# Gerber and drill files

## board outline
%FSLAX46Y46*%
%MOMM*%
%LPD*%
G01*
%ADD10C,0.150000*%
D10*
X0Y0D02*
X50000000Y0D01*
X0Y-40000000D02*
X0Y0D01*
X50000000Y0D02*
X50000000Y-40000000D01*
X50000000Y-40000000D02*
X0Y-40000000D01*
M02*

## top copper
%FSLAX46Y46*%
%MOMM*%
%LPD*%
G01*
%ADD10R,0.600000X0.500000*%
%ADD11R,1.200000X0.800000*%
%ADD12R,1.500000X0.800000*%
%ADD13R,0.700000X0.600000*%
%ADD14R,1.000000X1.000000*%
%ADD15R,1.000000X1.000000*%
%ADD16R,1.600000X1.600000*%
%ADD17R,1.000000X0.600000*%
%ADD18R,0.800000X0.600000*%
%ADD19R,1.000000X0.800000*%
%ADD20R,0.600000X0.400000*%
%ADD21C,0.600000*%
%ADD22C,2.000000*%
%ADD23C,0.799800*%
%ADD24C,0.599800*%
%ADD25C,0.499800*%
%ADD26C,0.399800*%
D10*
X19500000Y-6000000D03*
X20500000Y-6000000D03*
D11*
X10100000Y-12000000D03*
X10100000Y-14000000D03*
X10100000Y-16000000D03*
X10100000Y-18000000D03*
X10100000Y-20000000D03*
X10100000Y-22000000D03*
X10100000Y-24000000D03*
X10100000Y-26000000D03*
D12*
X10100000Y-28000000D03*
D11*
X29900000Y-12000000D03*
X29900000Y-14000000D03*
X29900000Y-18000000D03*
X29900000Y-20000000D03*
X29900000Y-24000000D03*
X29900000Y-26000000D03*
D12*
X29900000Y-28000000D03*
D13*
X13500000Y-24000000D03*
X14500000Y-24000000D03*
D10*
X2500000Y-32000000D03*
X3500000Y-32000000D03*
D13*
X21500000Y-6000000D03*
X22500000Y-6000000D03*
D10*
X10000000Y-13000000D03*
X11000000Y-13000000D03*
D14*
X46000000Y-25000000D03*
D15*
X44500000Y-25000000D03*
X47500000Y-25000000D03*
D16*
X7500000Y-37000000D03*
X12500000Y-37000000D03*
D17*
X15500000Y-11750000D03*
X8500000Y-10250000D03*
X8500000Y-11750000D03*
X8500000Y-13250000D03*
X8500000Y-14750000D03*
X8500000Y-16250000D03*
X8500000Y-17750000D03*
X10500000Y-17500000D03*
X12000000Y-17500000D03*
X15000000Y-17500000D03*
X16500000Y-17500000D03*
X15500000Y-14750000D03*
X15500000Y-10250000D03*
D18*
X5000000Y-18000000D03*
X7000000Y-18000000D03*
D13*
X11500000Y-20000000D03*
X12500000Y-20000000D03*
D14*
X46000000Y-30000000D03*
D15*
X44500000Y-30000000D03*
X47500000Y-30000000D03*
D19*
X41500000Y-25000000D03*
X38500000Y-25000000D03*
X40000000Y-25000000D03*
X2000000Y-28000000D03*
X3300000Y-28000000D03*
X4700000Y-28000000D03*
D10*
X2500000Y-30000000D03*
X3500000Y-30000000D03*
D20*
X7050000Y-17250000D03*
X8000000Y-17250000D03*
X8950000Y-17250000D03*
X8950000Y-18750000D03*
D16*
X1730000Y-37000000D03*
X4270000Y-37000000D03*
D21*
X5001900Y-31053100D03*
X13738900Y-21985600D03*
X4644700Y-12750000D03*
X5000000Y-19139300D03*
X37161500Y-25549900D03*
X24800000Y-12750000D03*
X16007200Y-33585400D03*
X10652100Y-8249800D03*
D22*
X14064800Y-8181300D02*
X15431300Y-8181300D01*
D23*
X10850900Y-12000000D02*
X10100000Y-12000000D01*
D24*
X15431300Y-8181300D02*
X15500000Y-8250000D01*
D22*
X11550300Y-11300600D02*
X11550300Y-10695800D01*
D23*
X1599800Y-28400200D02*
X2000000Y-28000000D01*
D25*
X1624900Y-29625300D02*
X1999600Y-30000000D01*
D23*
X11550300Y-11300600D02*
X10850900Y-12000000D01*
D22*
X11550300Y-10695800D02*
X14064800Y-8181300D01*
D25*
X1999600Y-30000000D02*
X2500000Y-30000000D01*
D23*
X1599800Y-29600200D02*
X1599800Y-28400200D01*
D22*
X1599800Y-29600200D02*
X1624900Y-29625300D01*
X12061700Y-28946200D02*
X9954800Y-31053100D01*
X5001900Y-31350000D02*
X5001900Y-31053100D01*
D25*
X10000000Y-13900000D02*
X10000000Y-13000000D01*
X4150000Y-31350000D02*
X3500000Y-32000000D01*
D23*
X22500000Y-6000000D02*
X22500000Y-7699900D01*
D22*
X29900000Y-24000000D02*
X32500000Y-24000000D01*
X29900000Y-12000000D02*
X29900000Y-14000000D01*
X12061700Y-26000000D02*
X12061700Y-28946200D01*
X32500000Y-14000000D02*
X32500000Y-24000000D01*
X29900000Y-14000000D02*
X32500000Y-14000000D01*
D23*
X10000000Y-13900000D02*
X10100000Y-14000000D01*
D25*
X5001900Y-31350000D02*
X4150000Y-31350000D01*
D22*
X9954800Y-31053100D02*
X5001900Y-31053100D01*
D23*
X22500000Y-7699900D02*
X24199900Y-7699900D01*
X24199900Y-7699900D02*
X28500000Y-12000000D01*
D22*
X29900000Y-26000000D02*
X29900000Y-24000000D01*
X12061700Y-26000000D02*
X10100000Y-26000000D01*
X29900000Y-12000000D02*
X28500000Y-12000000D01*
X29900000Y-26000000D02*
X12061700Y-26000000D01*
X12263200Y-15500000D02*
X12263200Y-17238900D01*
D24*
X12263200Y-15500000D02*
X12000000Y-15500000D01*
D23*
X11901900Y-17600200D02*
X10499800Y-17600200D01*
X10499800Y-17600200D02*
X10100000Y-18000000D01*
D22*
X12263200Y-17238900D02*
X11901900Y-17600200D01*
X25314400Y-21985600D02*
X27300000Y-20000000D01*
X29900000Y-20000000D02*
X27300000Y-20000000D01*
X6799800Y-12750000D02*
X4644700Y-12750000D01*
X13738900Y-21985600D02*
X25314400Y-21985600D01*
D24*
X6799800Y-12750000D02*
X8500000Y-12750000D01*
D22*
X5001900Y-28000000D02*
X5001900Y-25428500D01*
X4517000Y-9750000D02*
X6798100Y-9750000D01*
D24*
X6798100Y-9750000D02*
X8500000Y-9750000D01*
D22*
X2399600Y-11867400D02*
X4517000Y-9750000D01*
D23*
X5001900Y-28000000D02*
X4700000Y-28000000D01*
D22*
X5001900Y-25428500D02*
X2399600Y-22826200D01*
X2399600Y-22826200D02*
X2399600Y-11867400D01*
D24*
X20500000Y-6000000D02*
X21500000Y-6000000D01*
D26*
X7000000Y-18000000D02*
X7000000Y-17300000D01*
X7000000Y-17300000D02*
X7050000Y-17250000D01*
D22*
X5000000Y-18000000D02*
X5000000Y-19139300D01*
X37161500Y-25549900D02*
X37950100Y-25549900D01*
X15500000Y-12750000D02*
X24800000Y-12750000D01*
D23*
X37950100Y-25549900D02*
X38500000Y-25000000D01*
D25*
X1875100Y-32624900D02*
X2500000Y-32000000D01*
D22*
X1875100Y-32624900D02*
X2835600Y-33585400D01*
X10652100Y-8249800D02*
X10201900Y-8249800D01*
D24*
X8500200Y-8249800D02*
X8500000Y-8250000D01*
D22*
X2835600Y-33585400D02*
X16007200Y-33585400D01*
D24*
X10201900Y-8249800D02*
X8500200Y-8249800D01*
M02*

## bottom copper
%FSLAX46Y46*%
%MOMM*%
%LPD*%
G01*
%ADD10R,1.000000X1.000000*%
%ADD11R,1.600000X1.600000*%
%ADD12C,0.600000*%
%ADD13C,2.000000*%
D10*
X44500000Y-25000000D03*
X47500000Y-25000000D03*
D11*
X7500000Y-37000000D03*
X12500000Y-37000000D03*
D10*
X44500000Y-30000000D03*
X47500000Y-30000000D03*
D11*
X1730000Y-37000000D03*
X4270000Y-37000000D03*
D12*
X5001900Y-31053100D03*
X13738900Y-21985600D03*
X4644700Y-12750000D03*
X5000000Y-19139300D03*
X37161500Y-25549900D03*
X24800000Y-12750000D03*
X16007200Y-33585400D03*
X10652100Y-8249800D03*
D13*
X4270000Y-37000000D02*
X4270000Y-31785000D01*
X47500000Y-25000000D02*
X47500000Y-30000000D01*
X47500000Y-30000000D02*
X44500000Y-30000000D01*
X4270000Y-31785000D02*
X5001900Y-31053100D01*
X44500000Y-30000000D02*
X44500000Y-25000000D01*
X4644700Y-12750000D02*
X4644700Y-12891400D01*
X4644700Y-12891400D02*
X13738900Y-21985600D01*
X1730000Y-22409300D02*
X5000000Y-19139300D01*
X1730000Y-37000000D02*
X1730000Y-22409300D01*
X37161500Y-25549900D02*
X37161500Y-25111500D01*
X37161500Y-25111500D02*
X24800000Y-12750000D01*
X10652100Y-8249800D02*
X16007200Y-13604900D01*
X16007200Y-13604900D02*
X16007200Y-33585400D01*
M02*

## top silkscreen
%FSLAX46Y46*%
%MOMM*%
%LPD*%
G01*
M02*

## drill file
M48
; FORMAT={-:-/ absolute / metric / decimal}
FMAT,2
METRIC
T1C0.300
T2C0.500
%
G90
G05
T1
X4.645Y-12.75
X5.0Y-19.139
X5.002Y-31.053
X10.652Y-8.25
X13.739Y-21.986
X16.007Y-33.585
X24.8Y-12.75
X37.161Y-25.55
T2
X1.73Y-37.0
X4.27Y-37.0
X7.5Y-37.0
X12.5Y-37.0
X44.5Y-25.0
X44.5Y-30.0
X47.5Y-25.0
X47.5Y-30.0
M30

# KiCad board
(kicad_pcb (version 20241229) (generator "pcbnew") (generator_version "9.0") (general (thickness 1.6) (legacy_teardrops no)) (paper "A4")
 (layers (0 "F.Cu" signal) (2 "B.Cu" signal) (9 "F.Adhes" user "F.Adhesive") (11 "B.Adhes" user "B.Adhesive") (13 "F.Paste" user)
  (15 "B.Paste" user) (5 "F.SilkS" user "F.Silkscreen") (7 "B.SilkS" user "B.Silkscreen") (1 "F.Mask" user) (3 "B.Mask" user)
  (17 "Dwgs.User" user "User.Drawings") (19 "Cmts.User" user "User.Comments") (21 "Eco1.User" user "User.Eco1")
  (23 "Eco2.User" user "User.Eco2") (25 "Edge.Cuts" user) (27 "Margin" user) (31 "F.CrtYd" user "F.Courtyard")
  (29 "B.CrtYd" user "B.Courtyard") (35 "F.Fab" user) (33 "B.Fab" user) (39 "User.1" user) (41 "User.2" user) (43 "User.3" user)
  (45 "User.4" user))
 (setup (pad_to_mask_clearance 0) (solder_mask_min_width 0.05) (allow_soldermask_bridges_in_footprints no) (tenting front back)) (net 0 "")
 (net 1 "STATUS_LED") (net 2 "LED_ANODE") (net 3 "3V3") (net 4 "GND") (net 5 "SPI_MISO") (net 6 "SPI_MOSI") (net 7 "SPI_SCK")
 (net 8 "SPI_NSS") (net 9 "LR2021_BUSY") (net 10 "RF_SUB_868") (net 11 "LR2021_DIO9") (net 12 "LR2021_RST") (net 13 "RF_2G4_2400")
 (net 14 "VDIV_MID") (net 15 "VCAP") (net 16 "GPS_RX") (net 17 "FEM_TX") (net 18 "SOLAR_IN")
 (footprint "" (layer "F.Cu") (at 20 6)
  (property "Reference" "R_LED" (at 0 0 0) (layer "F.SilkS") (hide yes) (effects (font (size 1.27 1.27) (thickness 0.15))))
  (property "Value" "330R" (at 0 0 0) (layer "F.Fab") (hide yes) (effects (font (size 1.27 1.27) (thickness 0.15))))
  (pad "1" smd rect (at -0.5 0) (size 0.6 0.5) (layers "F.Cu" "F.Mask") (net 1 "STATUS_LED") (thermal_bridge_angle 45))
  (pad "2" smd rect (at 0.5 0) (size 0.6 0.5) (layers "F.Cu" "F.Mask") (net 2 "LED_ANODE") (thermal_bridge_angle 45)))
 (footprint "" (layer "F.Cu") (at 20 20)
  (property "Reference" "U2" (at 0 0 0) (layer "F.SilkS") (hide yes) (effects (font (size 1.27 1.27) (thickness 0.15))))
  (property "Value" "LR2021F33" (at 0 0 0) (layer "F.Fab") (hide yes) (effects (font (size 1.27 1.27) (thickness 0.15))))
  (pad "1" smd rect (at -9.9 -8) (size 1.2 0.8) (layers "F.Cu" "F.Mask") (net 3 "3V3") (thermal_bridge_angle 45))
  (pad "2" smd rect (at -9.9 -6) (size 1.2 0.8) (layers "F.Cu" "F.Mask") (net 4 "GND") (thermal_bridge_angle 45))
  (pad "3" smd rect (at -9.9 -4) (size 1.2 0.8) (layers "F.Cu" "F.Mask") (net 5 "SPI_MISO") (thermal_bridge_angle 45))
  (pad "4" smd rect (at -9.9 -2) (size 1.2 0.8) (layers "F.Cu" "F.Mask") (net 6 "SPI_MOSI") (thermal_bridge_angle 45))
  (pad "5" smd rect (at -9.9 0) (size 1.2 0.8) (layers "F.Cu" "F.Mask") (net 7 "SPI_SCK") (thermal_bridge_angle 45))
  (pad "6" smd rect (at -9.9 2) (size 1.2 0.8) (layers "F.Cu" "F.Mask") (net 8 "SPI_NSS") (thermal_bridge_angle 45))
  (pad "7" smd rect (at -9.9 4) (size 1.2 0.8) (layers "F.Cu" "F.Mask") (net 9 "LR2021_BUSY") (thermal_bridge_angle 45))
  (pad "8" smd rect (at -9.9 6) (size 1.2 0.8) (layers "F.Cu" "F.Mask") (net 4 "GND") (thermal_bridge_angle 45))
  (pad "9" smd rect (at -9.9 8) (size 1.5 0.8) (layers "F.Cu" "F.Mask") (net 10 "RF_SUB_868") (thermal_bridge_angle 45))
  (pad "10" smd rect (at 9.9 -8) (size 1.2 0.8) (layers "F.Cu" "F.Mask") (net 4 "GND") (thermal_bridge_angle 45))
  (pad "11" smd rect (at 9.9 -6) (size 1.2 0.8) (layers "F.Cu" "F.Mask") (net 4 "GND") (thermal_bridge_angle 45))
  (pad "13" smd rect (at 9.9 -2) (size 1.2 0.8) (layers "F.Cu" "F.Mask") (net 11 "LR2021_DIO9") (thermal_bridge_angle 45))
  (pad "14" smd rect (at 9.9 0) (size 1.2 0.8) (layers "F.Cu" "F.Mask") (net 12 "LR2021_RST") (thermal_bridge_angle 45))
  (pad "16" smd rect (at 9.9 4) (size 1.2 0.8) (layers "F.Cu" "F.Mask") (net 4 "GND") (thermal_bridge_angle 45))
  (pad "17" smd rect (at 9.9 6) (size 1.2 0.8) (layers "F.Cu" "F.Mask") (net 4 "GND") (thermal_bridge_angle 45))
  (pad "18" smd rect (at 9.9 8) (size 1.5 0.8) (layers "F.Cu" "F.Mask") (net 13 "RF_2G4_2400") (thermal_bridge_angle 45)))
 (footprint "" (layer "F.Cu") (at 14 24)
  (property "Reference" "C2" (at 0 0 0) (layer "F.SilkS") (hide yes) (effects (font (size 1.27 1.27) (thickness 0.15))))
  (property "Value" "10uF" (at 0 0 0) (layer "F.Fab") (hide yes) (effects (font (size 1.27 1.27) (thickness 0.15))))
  (pad "1" smd rect (at -0.5 0) (size 0.7 0.6) (layers "F.Cu" "F.Mask") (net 3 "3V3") (thermal_bridge_angle 45))
  (pad "2" smd rect (at 0.5 0) (size 0.7 0.6) (layers "F.Cu" "F.Mask") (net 4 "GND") (thermal_bridge_angle 45)))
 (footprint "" (layer "F.Cu") (at 3 32)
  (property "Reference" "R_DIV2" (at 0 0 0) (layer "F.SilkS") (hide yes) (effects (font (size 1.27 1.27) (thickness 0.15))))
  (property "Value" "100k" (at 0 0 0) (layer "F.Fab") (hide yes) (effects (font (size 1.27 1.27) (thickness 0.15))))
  (pad "1" smd rect (at -0.5 0) (size 0.6 0.5) (layers "F.Cu" "F.Mask") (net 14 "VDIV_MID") (thermal_bridge_angle 45))
  (pad "2" smd rect (at 0.5 0) (size 0.6 0.5) (layers "F.Cu" "F.Mask") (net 4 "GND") (thermal_bridge_angle 45)))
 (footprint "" (layer "F.Cu") (at 22 6)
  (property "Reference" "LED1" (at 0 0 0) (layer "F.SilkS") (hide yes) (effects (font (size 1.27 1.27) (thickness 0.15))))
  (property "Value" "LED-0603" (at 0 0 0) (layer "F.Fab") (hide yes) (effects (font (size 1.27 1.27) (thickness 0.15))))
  (pad "A" smd rect (at -0.5 0) (size 0.7 0.6) (layers "F.Cu" "F.Mask") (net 2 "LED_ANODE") (thermal_bridge_angle 45))
  (pad "K" smd rect (at 0.5 0) (size 0.7 0.6) (layers "F.Cu" "F.Mask") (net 4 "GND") (thermal_bridge_angle 45)))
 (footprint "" (layer "F.Cu") (at 10.5 13)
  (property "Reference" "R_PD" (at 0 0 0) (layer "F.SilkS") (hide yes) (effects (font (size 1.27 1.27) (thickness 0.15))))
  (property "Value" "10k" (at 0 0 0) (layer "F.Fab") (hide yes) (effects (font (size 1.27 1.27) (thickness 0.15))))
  (pad "1" smd rect (at -0.5 0) (size 0.6 0.5) (layers "F.Cu" "F.Mask") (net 4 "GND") (thermal_bridge_angle 45))
  (pad "2" smd rect (at 0.5 0) (size 0.6 0.5) (layers "F.Cu" "F.Mask") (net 5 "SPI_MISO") (thermal_bridge_angle 45)))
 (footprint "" (layer "F.Cu") (at 46 25)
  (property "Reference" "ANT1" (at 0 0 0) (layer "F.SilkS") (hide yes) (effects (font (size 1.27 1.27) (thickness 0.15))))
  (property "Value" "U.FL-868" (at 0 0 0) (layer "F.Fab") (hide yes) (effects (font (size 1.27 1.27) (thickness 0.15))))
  (pad "1" smd rect (at 0 0) (size 1 1) (layers "F.Cu" "F.Mask") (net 10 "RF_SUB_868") (thermal_bridge_angle 45))
  (pad "2" thru_hole rect (at -1.5 0) (size 1 1) (drill 0.5) (layers "*.Cu" "*.Mask") (remove_unused_layers no) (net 4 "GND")
   (thermal_bridge_angle 45))
  (pad "3" thru_hole rect (at 1.5 0) (size 1 1) (drill 0.5) (layers "*.Cu" "*.Mask") (remove_unused_layers no) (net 4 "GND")
   (thermal_bridge_angle 45)))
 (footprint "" (layer "F.Cu") (at 10 37)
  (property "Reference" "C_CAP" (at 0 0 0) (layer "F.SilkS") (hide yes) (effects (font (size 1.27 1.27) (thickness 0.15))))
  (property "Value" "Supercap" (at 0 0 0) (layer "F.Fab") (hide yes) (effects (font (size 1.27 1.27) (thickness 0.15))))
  (pad "1" thru_hole rect (at -2.5 0) (size 1.6 1.6) (drill 0.5) (layers "*.Cu" "*.Mask") (remove_unused_layers no) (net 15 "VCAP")
   (thermal_bridge_angle 45))
  (pad "2" thru_hole rect (at 2.5 0) (size 1.6 1.6) (drill 0.5) (layers "*.Cu" "*.Mask") (remove_unused_layers no) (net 4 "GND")
   (thermal_bridge_angle 45)))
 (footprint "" (layer "F.Cu") (at 12 14)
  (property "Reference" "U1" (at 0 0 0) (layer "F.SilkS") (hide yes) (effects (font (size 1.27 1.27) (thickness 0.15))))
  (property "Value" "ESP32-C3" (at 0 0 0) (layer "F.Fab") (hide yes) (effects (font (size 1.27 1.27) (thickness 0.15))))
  (pad "GND" smd rect (at 3.5 -2.25) (size 1 0.6) (layers "F.Cu" "F.Mask") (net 4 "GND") (thermal_bridge_angle 45))
  (pad "GPIO0" smd rect (at -3.5 -3.75) (size 1 0.6) (layers "F.Cu" "F.Mask") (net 14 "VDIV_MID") (thermal_bridge_angle 45))
  (pad "GPIO1" smd rect (at -3.5 -2.25) (size 1 0.6) (layers "F.Cu" "F.Mask") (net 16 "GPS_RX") (thermal_bridge_angle 45))
  (pad "GPIO2" smd rect (at -3.5 -0.75) (size 1 0.6) (layers "F.Cu" "F.Mask") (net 5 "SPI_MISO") (thermal_bridge_angle 45))
  (pad "GPIO3" smd rect (at -3.5 0.75) (size 1 0.6) (layers "F.Cu" "F.Mask") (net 12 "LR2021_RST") (thermal_bridge_angle 45))
  (pad "GPIO4" smd rect (at -3.5 2.25) (size 1 0.6) (layers "F.Cu" "F.Mask") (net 9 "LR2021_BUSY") (thermal_bridge_angle 45))
  (pad "GPIO5" smd rect (at -3.5 3.75) (size 1 0.6) (layers "F.Cu" "F.Mask") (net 11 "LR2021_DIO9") (thermal_bridge_angle 45))
  (pad "GPIO6" smd rect (at -1.5 3.5) (size 1 0.6) (layers "F.Cu" "F.Mask") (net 7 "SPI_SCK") (thermal_bridge_angle 45))
  (pad "GPIO7" smd rect (at 0 3.5) (size 1 0.6) (layers "F.Cu" "F.Mask") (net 6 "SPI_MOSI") (thermal_bridge_angle 45))
  (pad "GPIO9" smd rect (at 3 3.5) (size 1 0.6) (layers "F.Cu" "F.Mask") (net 1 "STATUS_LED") (thermal_bridge_angle 45))
  (pad "GPIO10" smd rect (at 4.5 3.5) (size 1 0.6) (layers "F.Cu" "F.Mask") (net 8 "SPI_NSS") (thermal_bridge_angle 45))
  (pad "GPIO19" smd rect (at 3.5 0.75) (size 1 0.6) (layers "F.Cu" "F.Mask") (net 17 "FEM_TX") (thermal_bridge_angle 45))
  (pad "VCC" smd rect (at 3.5 -3.75) (size 1 0.6) (layers "F.Cu" "F.Mask") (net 3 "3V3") (thermal_bridge_angle 45)))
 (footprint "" (layer "F.Cu") (at 6 18)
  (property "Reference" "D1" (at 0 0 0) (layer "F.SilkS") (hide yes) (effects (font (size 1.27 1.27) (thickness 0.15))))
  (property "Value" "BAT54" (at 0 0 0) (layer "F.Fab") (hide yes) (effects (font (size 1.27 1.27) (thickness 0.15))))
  (pad "A" smd rect (at -1 0) (size 0.8 0.6) (layers "F.Cu" "F.Mask") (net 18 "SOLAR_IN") (thermal_bridge_angle 45))
  (pad "K" smd rect (at 1 0) (size 0.8 0.6) (layers "F.Cu" "F.Mask") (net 15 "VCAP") (thermal_bridge_angle 45)))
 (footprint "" (layer "F.Cu") (at 12 20)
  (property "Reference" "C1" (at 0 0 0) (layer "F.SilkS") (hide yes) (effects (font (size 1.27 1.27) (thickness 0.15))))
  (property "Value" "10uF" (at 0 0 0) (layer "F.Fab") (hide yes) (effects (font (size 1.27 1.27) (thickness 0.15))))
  (pad "1" smd rect (at -0.5 0) (size 0.7 0.6) (layers "F.Cu" "F.Mask") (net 15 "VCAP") (thermal_bridge_angle 45))
  (pad "2" smd rect (at 0.5 0) (size 0.7 0.6) (layers "F.Cu" "F.Mask") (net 4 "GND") (thermal_bridge_angle 45)))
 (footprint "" (layer "F.Cu") (at 46 30)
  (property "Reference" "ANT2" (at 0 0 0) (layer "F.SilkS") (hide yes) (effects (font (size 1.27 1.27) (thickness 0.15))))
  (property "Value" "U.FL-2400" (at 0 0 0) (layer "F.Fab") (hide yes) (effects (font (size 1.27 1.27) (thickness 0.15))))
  (pad "1" smd rect (at 0 0) (size 1 1) (layers "F.Cu" "F.Mask") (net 13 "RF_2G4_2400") (thermal_bridge_angle 45))
  (pad "2" thru_hole rect (at -1.5 0) (size 1 1) (drill 0.5) (layers "*.Cu" "*.Mask") (remove_unused_layers no) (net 4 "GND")
   (thermal_bridge_angle 45))
  (pad "3" thru_hole rect (at 1.5 0) (size 1 1) (drill 0.5) (layers "*.Cu" "*.Mask") (remove_unused_layers no) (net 4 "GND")
   (thermal_bridge_angle 45)))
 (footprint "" (layer "F.Cu") (at 40 25)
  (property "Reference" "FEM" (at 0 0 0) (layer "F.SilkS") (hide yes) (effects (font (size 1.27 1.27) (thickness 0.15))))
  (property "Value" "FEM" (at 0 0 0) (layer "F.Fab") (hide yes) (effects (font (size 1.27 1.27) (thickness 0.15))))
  (pad "GND" smd rect (at 1.5 0) (size 1 0.8) (layers "F.Cu" "F.Mask") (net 4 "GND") (thermal_bridge_angle 45))
  (pad "TX" smd rect (at -1.5 0) (size 1 0.8) (layers "F.Cu" "F.Mask") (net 17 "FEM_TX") (thermal_bridge_angle 45))
  (pad "VCC" smd rect (at 0 0) (size 1 0.8) (layers "F.Cu" "F.Mask") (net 3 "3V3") (thermal_bridge_angle 45)))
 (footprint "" (layer "F.Cu") (at 4 28)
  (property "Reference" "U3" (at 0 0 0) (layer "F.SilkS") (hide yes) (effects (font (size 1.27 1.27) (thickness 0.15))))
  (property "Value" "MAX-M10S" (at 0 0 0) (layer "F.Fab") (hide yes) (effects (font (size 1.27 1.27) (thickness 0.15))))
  (pad "1" smd rect (at -2 0) (size 1 0.8) (layers "F.Cu" "F.Mask") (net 3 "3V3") (thermal_bridge_angle 45))
  (pad "2" smd rect (at -0.7 0) (size 1 0.8) (layers "F.Cu" "F.Mask") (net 4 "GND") (thermal_bridge_angle 45))
  (pad "3" smd rect (at 0.7 0) (size 1 0.8) (layers "F.Cu" "F.Mask") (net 16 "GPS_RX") (thermal_bridge_angle 45)))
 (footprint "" (layer "F.Cu") (at 3 30)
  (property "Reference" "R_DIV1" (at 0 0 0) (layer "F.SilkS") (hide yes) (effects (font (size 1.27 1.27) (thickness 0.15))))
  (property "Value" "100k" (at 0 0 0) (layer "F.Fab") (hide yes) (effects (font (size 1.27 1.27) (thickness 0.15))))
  (pad "1" smd rect (at -0.5 0) (size 0.6 0.5) (layers "F.Cu" "F.Mask") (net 3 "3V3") (thermal_bridge_angle 45))
  (pad "2" smd rect (at 0.5 0) (size 0.6 0.5) (layers "F.Cu" "F.Mask") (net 14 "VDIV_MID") (thermal_bridge_angle 45)))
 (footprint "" (layer "F.Cu") (at 8 18)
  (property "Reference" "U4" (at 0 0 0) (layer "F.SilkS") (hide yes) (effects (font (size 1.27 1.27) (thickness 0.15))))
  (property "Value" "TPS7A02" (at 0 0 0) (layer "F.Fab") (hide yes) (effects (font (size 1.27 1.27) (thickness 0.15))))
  (pad "1" smd rect (at -0.95 -0.75) (size 0.6 0.4) (layers "F.Cu" "F.Mask") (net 15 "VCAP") (thermal_bridge_angle 45))
  (pad "2" smd rect (at 0 -0.75) (size 0.6 0.4) (layers "F.Cu" "F.Mask") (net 4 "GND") (thermal_bridge_angle 45))
  (pad "3" smd rect (at 0.95 -0.75) (size 0.6 0.4) (layers "F.Cu" "F.Mask") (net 15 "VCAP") (thermal_bridge_angle 45))
  (pad "4" smd rect (at 0.95 0.75) (size 0.6 0.4) (layers "F.Cu" "F.Mask") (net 3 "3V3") (thermal_bridge_angle 45)))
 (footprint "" (layer "F.Cu") (at 3 37)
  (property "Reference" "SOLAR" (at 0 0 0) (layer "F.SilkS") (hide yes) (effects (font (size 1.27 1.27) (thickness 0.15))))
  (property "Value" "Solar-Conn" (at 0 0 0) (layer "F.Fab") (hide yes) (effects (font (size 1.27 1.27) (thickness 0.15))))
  (pad "1" thru_hole rect (at -1.27 0) (size 1.6 1.6) (drill 0.5) (layers "*.Cu" "*.Mask") (remove_unused_layers no) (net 18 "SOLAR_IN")
   (thermal_bridge_angle 45))
  (pad "2" thru_hole rect (at 1.27 0) (size 1.6 1.6) (drill 0.5) (layers "*.Cu" "*.Mask") (remove_unused_layers no) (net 4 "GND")
   (thermal_bridge_angle 45)))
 (gr_line (start 0 0) (end 50 0) (stroke (width 0.15) (type default)) (layer "Edge.Cuts"))
 (gr_line (start 0 40) (end 0 0) (stroke (width 0.15) (type default)) (layer "Edge.Cuts"))
 (gr_line (start 50 0) (end 50 40) (stroke (width 0.15) (type default)) (layer "Edge.Cuts"))
 (gr_line (start 50 40) (end 0 40) (stroke (width 0.15) (type default)) (layer "Edge.Cuts"))
 (segment (start 14.0648 8.1813) (end 15.4313 8.1813) (width 2) (layer "F.Cu") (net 3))
 (segment (start 10.8509 12) (end 10.1 12) (width 0.7998) (layer "F.Cu") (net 3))
 (segment (start 15.4313 8.1813) (end 15.5 8.25) (width 0.5998) (layer "F.Cu") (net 3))
 (segment (start 11.5503 11.3006) (end 11.5503 10.6958) (width 2) (layer "F.Cu") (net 3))
 (segment (start 1.5998 28.4002) (end 2 28) (width 0.7998) (layer "F.Cu") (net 3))
 (segment (start 1.6249 29.6253) (end 1.9996 30) (width 0.4998) (layer "F.Cu") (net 3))
 (segment (start 11.5503 11.3006) (end 10.8509 12) (width 0.7998) (layer "F.Cu") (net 3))
 (segment (start 11.5503 10.6958) (end 14.0648 8.1813) (width 2) (layer "F.Cu") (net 3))
 (segment (start 1.9996 30) (end 2.5 30) (width 0.4998) (layer "F.Cu") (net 3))
 (segment (start 1.5998 29.6002) (end 1.5998 28.4002) (width 0.7998) (layer "F.Cu") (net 3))
 (segment (start 1.5998 29.6002) (end 1.6249 29.6253) (width 2) (layer "F.Cu") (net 3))
 (segment (start 12.0617 28.9462) (end 9.9548 31.0531) (width 2) (layer "F.Cu") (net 4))
 (segment (start 5.0019 31.35) (end 5.0019 31.0531) (width 2) (layer "F.Cu") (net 4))
 (segment (start 10 13.9) (end 10 13) (width 0.4998) (layer "F.Cu") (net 4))
 (segment (start 4.15 31.35) (end 3.5 32) (width 0.4998) (layer "F.Cu") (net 4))
 (segment (start 22.5 6) (end 22.5 7.6999) (width 0.7998) (layer "F.Cu") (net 4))
 (segment (start 29.9 24) (end 32.5 24) (width 2) (layer "F.Cu") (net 4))
 (segment (start 29.9 12) (end 29.9 14) (width 2) (layer "F.Cu") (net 4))
 (segment (start 12.0617 26) (end 12.0617 28.9462) (width 2) (layer "F.Cu") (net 4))
 (segment (start 32.5 14) (end 32.5 24) (width 2) (layer "F.Cu") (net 4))
 (segment (start 29.9 14) (end 32.5 14) (width 2) (layer "F.Cu") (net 4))
 (segment (start 10 13.9) (end 10.1 14) (width 0.7998) (layer "F.Cu") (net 4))
 (segment (start 5.0019 31.35) (end 4.15 31.35) (width 0.4998) (layer "F.Cu") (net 4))
 (segment (start 9.9548 31.0531) (end 5.0019 31.0531) (width 2) (layer "F.Cu") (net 4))
 (segment (start 22.5 7.6999) (end 24.1999 7.6999) (width 0.7998) (layer "F.Cu") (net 4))
 (segment (start 24.1999 7.6999) (end 28.5 12) (width 0.7998) (layer "F.Cu") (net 4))
 (segment (start 29.9 26) (end 29.9 24) (width 2) (layer "F.Cu") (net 4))
 (segment (start 12.0617 26) (end 10.1 26) (width 2) (layer "F.Cu") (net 4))
 (segment (start 29.9 12) (end 28.5 12) (width 2) (layer "F.Cu") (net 4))
 (segment (start 29.9 26) (end 12.0617 26) (width 2) (layer "F.Cu") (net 4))
 (via (at 5.0019 31.0531) (size 0.6) (drill 0.3) (layers "F.Cu" "B.Cu") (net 4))
 (segment (start 4.27 37) (end 4.27 31.785) (width 2) (layer "B.Cu") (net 4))
 (segment (start 47.5 25) (end 47.5 30) (width 2) (layer "B.Cu") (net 4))
 (segment (start 47.5 30) (end 44.5 30) (width 2) (layer "B.Cu") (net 4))
 (segment (start 4.27 31.785) (end 5.0019 31.0531) (width 2) (layer "B.Cu") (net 4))
 (segment (start 44.5 30) (end 44.5 25) (width 2) (layer "B.Cu") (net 4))
 (segment (start 12.2632 15.5) (end 12.2632 17.2389) (width 2) (layer "F.Cu") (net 6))
 (segment (start 12.2632 15.5) (end 12 15.5) (width 0.5998) (layer "F.Cu") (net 6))
 (segment (start 11.9019 17.6002) (end 10.4998 17.6002) (width 0.7998) (layer "F.Cu") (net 6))
 (segment (start 10.4998 17.6002) (end 10.1 18) (width 0.7998) (layer "F.Cu") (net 6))
 (segment (start 12.2632 17.2389) (end 11.9019 17.6002) (width 2) (layer "F.Cu") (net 6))
 (segment (start 25.3144 21.9856) (end 27.3 20) (width 2) (layer "F.Cu") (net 12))
 (segment (start 29.9 20) (end 27.3 20) (width 2) (layer "F.Cu") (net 12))
 (segment (start 6.7998 12.75) (end 4.6447 12.75) (width 2) (layer "F.Cu") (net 12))
 (segment (start 13.7389 21.9856) (end 25.3144 21.9856) (width 2) (layer "F.Cu") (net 12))
 (segment (start 6.7998 12.75) (end 8.5 12.75) (width 0.5998) (layer "F.Cu") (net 12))
 (via (at 13.7389 21.9856) (size 0.6) (drill 0.3) (layers "F.Cu" "B.Cu") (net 12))
 (via (at 4.6447 12.75) (size 0.6) (drill 0.3) (layers "F.Cu" "B.Cu") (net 12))
 (segment (start 4.6447 12.75) (end 4.6447 12.8914) (width 2) (layer "B.Cu") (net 12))
 (segment (start 4.6447 12.8914) (end 13.7389 21.9856) (width 2) (layer "B.Cu") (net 12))
 (segment (start 5.0019 28) (end 5.0019 25.4285) (width 2) (layer "F.Cu") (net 16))
 (segment (start 4.517 9.75) (end 6.7981 9.75) (width 2) (layer "F.Cu") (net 16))
 (segment (start 6.7981 9.75) (end 8.5 9.75) (width 0.5998) (layer "F.Cu") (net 16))
 (segment (start 2.3996 11.8674) (end 4.517 9.75) (width 2) (layer "F.Cu") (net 16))
 (segment (start 5.0019 28) (end 4.7 28) (width 0.7998) (layer "F.Cu") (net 16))
 (segment (start 5.0019 25.4285) (end 2.3996 22.8262) (width 2) (layer "F.Cu") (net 16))
 (segment (start 2.3996 22.8262) (end 2.3996 11.8674) (width 2) (layer "F.Cu") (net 16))
 (segment (start 20.5 6) (end 21.5 6) (width 0.5998) (layer "F.Cu") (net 2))
 (segment (start 7 18) (end 7 17.3) (width 0.3998) (layer "F.Cu") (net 15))
 (segment (start 7 17.3) (end 7.05 17.25) (width 0.3998) (layer "F.Cu") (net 15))
 (segment (start 5 18) (end 5 19.1393) (width 2) (layer "F.Cu") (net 18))
 (via (at 5 19.1393) (size 0.6) (drill 0.3) (layers "F.Cu" "B.Cu") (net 18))
 (segment (start 1.73 22.4093) (end 5 19.1393) (width 2) (layer "B.Cu") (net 18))
 (segment (start 1.73 37) (end 1.73 22.4093) (width 2) (layer "B.Cu") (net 18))
 (segment (start 37.1615 25.5499) (end 37.9501 25.5499) (width 2) (layer "F.Cu") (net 17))
 (segment (start 15.5 12.75) (end 24.8 12.75) (width 2) (layer "F.Cu") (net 17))
 (segment (start 37.9501 25.5499) (end 38.5 25) (width 0.7998) (layer "F.Cu") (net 17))
 (via (at 37.1615 25.5499) (size 0.6) (drill 0.3) (layers "F.Cu" "B.Cu") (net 17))
 (via (at 24.8 12.75) (size 0.6) (drill 0.3) (layers "F.Cu" "B.Cu") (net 17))
 (segment (start 37.1615 25.5499) (end 37.1615 25.1115) (width 2) (layer "B.Cu") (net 17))
 (segment (start 37.1615 25.1115) (end 24.8 12.75) (width 2) (layer "B.Cu") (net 17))
 (segment (start 1.8751 32.6249) (end 2.5 32) (width 0.4998) (layer "F.Cu") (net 14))
 (segment (start 1.8751 32.6249) (end 2.8356 33.5854) (width 2) (layer "F.Cu") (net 14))
 (segment (start 10.6521 8.2498) (end 10.2019 8.2498) (width 2) (layer "F.Cu") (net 14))
 (segment (start 8.5002 8.2498) (end 8.5 8.25) (width 0.5998) (layer "F.Cu") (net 14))
 (segment (start 2.8356 33.5854) (end 16.0072 33.5854) (width 2) (layer "F.Cu") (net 14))
 (segment (start 10.2019 8.2498) (end 8.5002 8.2498) (width 0.5998) (layer "F.Cu") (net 14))
 (via (at 16.0072 33.5854) (size 0.6) (drill 0.3) (layers "F.Cu" "B.Cu") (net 14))
 (via (at 10.6521 8.2498) (size 0.6) (drill 0.3) (layers "F.Cu" "B.Cu") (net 14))
 (segment (start 10.6521 8.2498) (end 16.0072 13.6049) (width 2) (layer "B.Cu") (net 14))
 (segment (start 16.0072 13.6049) (end 16.0072 33.5854) (width 2) (layer "B.Cu") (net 14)))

